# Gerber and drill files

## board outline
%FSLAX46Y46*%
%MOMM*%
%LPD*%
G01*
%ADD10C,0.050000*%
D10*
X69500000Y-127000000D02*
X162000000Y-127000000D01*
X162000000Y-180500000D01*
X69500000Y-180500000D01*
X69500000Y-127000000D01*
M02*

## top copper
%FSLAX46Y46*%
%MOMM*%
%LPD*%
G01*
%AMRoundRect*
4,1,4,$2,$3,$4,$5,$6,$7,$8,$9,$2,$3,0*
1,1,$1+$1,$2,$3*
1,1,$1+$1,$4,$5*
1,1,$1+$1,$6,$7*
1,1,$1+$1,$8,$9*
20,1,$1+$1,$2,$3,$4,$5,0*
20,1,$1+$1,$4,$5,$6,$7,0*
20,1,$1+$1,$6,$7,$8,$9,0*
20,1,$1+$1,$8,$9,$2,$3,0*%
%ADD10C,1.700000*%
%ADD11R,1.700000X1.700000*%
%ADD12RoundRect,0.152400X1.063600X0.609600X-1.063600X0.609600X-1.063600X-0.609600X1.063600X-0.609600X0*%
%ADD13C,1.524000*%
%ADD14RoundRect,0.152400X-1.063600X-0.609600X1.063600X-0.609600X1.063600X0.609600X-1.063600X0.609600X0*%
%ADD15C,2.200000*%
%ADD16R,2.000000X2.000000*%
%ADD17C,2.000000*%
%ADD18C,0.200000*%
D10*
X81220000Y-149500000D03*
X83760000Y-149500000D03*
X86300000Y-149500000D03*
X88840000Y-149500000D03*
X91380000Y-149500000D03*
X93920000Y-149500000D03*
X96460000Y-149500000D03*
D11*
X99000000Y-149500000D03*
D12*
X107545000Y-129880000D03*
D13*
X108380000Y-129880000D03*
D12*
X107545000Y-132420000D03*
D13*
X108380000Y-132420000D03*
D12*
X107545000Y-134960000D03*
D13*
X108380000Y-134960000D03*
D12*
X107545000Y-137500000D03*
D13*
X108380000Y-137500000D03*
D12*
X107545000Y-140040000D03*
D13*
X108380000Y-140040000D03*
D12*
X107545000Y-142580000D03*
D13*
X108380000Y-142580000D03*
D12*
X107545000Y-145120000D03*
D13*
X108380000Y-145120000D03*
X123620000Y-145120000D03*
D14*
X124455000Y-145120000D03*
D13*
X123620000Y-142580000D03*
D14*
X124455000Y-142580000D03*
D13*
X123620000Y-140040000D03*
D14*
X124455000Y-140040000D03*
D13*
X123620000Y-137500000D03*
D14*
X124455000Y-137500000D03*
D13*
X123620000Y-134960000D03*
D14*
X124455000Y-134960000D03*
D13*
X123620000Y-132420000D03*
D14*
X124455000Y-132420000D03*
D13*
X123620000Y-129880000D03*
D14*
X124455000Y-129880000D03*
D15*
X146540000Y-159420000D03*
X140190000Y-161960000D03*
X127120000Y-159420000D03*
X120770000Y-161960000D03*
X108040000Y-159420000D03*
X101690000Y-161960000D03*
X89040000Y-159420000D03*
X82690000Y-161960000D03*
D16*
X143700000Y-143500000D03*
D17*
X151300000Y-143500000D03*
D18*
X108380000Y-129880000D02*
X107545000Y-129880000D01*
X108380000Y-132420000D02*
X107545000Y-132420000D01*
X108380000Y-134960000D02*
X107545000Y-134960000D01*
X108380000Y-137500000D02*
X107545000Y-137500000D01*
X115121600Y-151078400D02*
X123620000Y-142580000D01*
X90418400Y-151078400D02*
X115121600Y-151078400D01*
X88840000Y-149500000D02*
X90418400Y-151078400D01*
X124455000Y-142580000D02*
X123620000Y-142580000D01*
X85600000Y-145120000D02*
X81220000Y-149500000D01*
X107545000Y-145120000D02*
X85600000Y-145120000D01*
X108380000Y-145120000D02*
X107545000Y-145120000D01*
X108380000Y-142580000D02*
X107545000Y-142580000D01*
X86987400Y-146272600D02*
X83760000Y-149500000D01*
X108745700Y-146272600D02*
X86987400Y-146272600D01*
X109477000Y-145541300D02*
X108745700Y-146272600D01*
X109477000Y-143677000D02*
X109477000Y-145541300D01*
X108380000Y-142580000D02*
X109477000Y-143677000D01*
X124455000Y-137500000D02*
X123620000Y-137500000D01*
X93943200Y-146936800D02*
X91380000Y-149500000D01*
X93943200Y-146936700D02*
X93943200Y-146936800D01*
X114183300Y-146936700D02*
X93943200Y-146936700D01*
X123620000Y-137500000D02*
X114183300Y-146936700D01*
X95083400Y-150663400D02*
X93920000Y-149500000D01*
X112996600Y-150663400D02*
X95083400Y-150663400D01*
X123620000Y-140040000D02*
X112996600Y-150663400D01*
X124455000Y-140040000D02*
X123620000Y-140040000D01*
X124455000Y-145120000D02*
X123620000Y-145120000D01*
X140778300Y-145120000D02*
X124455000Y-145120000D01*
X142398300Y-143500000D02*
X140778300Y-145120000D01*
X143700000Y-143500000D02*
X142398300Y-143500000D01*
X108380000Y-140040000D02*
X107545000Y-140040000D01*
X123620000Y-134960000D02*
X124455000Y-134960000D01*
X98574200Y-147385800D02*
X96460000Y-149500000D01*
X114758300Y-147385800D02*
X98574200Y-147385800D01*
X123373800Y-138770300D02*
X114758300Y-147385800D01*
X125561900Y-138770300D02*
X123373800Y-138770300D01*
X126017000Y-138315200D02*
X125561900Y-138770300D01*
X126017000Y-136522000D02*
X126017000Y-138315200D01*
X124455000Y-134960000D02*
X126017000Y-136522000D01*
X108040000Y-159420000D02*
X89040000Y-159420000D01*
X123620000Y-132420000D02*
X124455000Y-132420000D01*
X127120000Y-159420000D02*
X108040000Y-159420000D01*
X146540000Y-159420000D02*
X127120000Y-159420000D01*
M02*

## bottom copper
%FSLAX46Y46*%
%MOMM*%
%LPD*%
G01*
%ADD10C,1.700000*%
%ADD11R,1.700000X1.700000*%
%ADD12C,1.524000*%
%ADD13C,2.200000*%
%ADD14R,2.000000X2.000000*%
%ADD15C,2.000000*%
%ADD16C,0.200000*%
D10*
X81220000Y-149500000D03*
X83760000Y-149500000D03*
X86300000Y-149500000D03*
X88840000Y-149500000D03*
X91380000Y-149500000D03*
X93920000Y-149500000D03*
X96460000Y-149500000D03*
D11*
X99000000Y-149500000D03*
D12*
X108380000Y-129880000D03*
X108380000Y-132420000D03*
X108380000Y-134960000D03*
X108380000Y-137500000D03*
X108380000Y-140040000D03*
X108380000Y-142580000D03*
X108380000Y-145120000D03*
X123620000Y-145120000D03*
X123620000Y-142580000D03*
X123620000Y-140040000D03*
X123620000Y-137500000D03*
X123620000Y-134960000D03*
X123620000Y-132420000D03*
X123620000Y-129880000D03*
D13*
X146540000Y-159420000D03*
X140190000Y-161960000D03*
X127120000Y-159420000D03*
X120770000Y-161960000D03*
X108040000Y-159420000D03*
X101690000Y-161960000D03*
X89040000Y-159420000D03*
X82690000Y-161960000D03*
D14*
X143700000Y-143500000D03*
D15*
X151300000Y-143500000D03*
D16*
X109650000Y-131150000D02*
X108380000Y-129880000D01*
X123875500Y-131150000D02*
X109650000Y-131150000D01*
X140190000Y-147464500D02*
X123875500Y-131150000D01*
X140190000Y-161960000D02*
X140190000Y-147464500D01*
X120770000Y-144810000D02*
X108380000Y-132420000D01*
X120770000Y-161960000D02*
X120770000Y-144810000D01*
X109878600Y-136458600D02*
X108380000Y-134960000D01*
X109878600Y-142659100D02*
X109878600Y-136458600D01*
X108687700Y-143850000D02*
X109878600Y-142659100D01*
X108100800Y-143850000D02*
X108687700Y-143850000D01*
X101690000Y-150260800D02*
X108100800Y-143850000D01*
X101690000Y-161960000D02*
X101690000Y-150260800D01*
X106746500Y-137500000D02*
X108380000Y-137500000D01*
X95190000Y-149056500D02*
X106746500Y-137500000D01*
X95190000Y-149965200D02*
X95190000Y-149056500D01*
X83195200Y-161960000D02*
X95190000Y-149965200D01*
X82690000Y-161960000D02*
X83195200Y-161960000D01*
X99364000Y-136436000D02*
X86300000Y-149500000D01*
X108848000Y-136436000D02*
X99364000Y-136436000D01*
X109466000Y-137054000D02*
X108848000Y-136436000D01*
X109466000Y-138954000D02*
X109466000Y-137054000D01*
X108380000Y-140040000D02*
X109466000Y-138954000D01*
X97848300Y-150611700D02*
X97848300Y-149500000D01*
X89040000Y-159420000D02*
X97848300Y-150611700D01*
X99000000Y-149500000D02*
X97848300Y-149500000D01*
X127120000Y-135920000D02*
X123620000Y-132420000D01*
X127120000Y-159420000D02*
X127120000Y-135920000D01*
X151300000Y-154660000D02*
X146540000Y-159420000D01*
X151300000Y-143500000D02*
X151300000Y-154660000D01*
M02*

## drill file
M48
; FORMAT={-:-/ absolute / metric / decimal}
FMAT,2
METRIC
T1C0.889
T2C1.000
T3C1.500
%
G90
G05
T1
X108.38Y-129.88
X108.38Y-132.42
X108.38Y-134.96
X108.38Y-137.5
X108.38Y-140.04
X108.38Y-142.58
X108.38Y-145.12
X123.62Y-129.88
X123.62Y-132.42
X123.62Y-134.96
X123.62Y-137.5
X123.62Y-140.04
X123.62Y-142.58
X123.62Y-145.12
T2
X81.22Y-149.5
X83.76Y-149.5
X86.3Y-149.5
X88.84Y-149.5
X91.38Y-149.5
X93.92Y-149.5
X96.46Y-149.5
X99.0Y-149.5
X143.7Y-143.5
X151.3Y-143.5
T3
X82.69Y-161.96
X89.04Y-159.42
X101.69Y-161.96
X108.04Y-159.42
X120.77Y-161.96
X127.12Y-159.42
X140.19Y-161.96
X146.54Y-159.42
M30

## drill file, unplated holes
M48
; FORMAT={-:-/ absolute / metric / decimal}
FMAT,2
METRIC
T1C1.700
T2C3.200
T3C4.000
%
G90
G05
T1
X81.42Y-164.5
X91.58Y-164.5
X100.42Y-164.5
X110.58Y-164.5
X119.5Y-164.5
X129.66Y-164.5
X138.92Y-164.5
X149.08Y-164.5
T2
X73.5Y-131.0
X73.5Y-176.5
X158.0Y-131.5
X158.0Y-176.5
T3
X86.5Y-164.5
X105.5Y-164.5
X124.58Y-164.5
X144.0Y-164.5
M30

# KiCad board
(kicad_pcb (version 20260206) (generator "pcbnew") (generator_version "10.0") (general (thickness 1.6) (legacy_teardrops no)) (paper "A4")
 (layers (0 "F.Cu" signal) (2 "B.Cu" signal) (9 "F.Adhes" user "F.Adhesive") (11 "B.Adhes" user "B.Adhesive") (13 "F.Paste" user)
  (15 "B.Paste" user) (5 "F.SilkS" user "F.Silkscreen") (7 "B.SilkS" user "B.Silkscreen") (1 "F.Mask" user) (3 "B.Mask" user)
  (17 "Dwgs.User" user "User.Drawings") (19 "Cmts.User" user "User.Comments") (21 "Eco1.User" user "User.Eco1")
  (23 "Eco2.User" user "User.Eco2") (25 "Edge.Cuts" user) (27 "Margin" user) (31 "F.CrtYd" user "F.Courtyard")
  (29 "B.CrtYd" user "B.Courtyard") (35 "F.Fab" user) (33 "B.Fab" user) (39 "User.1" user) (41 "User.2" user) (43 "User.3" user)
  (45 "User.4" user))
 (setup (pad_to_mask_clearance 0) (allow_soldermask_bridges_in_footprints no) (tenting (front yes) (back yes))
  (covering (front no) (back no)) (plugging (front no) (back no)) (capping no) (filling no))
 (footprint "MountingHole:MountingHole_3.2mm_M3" (layer "F.Cu") (at 158 176.5)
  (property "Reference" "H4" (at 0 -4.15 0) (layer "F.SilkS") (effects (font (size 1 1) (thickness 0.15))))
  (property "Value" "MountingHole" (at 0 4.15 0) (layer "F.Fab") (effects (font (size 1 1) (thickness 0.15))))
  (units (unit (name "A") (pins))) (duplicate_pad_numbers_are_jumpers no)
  (pad "" np_thru_hole circle (at 0 0) (size 3.2 3.2) (drill 3.2) (layers "*.Cu" "*.Mask")))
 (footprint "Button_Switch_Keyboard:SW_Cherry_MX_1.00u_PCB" (layer "F.Cu") (at 127.12 159.42)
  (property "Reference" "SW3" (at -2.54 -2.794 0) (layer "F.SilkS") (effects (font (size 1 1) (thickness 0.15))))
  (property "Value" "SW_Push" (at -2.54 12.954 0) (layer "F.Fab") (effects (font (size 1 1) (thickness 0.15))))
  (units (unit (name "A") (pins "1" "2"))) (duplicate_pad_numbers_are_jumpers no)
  (pad "" np_thru_hole circle (at -7.62 5.08) (size 1.7 1.7) (drill 1.7) (layers "*.Cu" "*.Mask"))
  (pad "" np_thru_hole circle (at -2.54 5.08) (size 4 4) (drill 4) (layers "*.Cu" "*.Mask"))
  (pad "" np_thru_hole circle (at 2.54 5.08) (size 1.7 1.7) (drill 1.7) (layers "*.Cu" "*.Mask"))
  (pad "1" thru_hole circle (at 0 0) (size 2.2 2.2) (drill 1.5) (layers "*.Cu" "*.Mask") (remove_unused_layers no) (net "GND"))
  (pad "2" thru_hole circle (at -6.35 2.54) (size 2.2 2.2) (drill 1.5) (layers "*.Cu" "*.Mask") (remove_unused_layers no) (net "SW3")))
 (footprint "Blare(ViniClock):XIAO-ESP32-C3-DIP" (layer "F.Cu") (at 116 137.5 90)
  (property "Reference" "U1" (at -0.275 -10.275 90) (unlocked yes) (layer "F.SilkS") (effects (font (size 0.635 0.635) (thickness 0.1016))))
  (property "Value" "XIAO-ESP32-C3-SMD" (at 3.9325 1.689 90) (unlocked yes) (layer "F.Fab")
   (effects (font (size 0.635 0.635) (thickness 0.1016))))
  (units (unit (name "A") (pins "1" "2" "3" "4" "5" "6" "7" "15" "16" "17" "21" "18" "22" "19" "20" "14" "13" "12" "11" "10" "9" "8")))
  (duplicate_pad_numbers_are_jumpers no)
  (pad "1" smd roundrect (at 7.62 -8.455 180) (size 2.432 1.524) (layers "F.Cu" "F.Mask") (roundrect_rratio 0.1) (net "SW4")
   (thermal_bridge_angle 45))
  (pad "1" thru_hole circle (at 7.62 -7.62 180) (size 1.524 1.524) (drill 0.889) (layers "*.Cu" "*.Mask") (remove_unused_layers no)
   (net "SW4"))
  (pad "2" smd roundrect (at 5.08 -8.455 180) (size 2.432 1.524) (layers "F.Cu" "F.Mask") (roundrect_rratio 0.1) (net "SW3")
   (thermal_bridge_angle 45))
  (pad "2" thru_hole circle (at 5.08 -7.62 180) (size 1.524 1.524) (drill 0.889) (layers "*.Cu" "*.Mask") (remove_unused_layers no)
   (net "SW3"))
  (pad "3" smd roundrect (at 2.54 -8.455 180) (size 2.432 1.524) (layers "F.Cu" "F.Mask") (roundrect_rratio 0.1) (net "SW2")
   (thermal_bridge_angle 45))
  (pad "3" thru_hole circle (at 2.54 -7.62 180) (size 1.524 1.524) (drill 0.889) (layers "*.Cu" "*.Mask") (remove_unused_layers no)
   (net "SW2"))
  (pad "4" smd roundrect (at 0 -8.455 180) (size 2.432 1.524) (layers "F.Cu" "F.Mask") (roundrect_rratio 0.1) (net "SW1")
   (thermal_bridge_angle 45))
  (pad "4" thru_hole circle (at 0 -7.62 180) (size 1.524 1.524) (drill 0.889) (layers "*.Cu" "*.Mask") (remove_unused_layers no) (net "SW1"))
  (pad "5" smd roundrect (at -2.54 -8.455 180) (size 2.432 1.524) (layers "F.Cu" "F.Mask") (roundrect_rratio 0.1) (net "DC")
   (thermal_bridge_angle 45))
  (pad "5" thru_hole circle (at -2.54 -7.62 180) (size 1.524 1.524) (drill 0.889) (layers "*.Cu" "*.Mask") (remove_unused_layers no)
   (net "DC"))
  (pad "6" smd roundrect (at -5.08 -8.455 180) (size 2.432 1.524) (layers "F.Cu" "F.Mask") (roundrect_rratio 0.1) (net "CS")
   (thermal_bridge_angle 45))
  (pad "6" thru_hole circle (at -5.08 -7.62 180) (size 1.524 1.524) (drill 0.889) (layers "*.Cu" "*.Mask") (remove_unused_layers no)
   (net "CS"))
  (pad "7" smd roundrect (at -7.62 -8.455 180) (size 2.432 1.524) (layers "F.Cu" "F.Mask") (roundrect_rratio 0.1) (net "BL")
   (thermal_bridge_angle 45))
  (pad "7" thru_hole circle (at -7.62 -7.62 180) (size 1.524 1.524) (drill 0.889) (layers "*.Cu" "*.Mask") (remove_unused_layers no)
   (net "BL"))
  (pad "8" thru_hole circle (at -7.62 7.62) (size 1.524 1.524) (drill 0.889) (layers "*.Cu" "*.Mask") (remove_unused_layers no)
   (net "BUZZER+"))
  (pad "8" smd roundrect (at -7.62 8.455) (size 2.432 1.524) (layers "F.Cu" "F.Mask") (roundrect_rratio 0.1) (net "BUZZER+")
   (thermal_bridge_angle 45))
  (pad "9" thru_hole circle (at -5.08 7.62) (size 1.524 1.524) (drill 0.889) (layers "*.Cu" "*.Mask") (remove_unused_layers no) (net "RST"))
  (pad "9" smd roundrect (at -5.08 8.455) (size 2.432 1.524) (layers "F.Cu" "F.Mask") (roundrect_rratio 0.1) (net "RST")
   (thermal_bridge_angle 45))
  (pad "10" thru_hole circle (at -2.54 7.62) (size 1.524 1.524) (drill 0.889) (layers "*.Cu" "*.Mask") (remove_unused_layers no) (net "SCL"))
  (pad "10" smd roundrect (at -2.54 8.455) (size 2.432 1.524) (layers "F.Cu" "F.Mask") (roundrect_rratio 0.1) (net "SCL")
   (thermal_bridge_angle 45))
  (pad "11" thru_hole circle (at 0 7.62) (size 1.524 1.524) (drill 0.889) (layers "*.Cu" "*.Mask") (remove_unused_layers no) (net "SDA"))
  (pad "11" smd roundrect (at 0 8.455) (size 2.432 1.524) (layers "F.Cu" "F.Mask") (roundrect_rratio 0.1) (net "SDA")
   (thermal_bridge_angle 45))
  (pad "12" thru_hole circle (at 2.54 7.62) (size 1.524 1.524) (drill 0.889) (layers "*.Cu" "*.Mask") (remove_unused_layers no) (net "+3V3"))
  (pad "12" smd roundrect (at 2.54 8.455) (size 2.432 1.524) (layers "F.Cu" "F.Mask") (roundrect_rratio 0.1) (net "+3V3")
   (thermal_bridge_angle 45))
  (pad "13" thru_hole circle (at 5.08 7.62) (size 1.524 1.524) (drill 0.889) (layers "*.Cu" "*.Mask") (remove_unused_layers no) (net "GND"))
  (pad "13" smd roundrect (at 5.08 8.455) (size 2.432 1.524) (layers "F.Cu" "F.Mask") (roundrect_rratio 0.1) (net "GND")
   (thermal_bridge_angle 45))
  (pad "14" thru_hole circle (at 7.62 7.62) (size 1.524 1.524) (drill 0.889) (layers "*.Cu" "*.Mask") (remove_unused_layers no)
   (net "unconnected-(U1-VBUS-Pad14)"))
  (pad "14" smd roundrect (at 7.62 8.455) (size 2.432 1.524) (layers "F.Cu" "F.Mask") (roundrect_rratio 0.1)
   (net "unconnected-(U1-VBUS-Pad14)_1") (thermal_bridge_angle 45)))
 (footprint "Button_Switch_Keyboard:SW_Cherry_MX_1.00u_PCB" (layer "F.Cu") (at 89.04 159.42)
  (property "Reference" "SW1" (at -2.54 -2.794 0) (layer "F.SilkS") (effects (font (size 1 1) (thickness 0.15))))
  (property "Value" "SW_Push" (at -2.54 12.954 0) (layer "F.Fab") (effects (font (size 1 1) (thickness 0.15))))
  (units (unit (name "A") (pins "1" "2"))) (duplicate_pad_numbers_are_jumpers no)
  (pad "" np_thru_hole circle (at -7.62 5.08) (size 1.7 1.7) (drill 1.7) (layers "*.Cu" "*.Mask"))
  (pad "" np_thru_hole circle (at -2.54 5.08) (size 4 4) (drill 4) (layers "*.Cu" "*.Mask"))
  (pad "" np_thru_hole circle (at 2.54 5.08) (size 1.7 1.7) (drill 1.7) (layers "*.Cu" "*.Mask"))
  (pad "1" thru_hole circle (at 0 0) (size 2.2 2.2) (drill 1.5) (layers "*.Cu" "*.Mask") (remove_unused_layers no) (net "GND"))
  (pad "2" thru_hole circle (at -6.35 2.54) (size 2.2 2.2) (drill 1.5) (layers "*.Cu" "*.Mask") (remove_unused_layers no) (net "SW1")))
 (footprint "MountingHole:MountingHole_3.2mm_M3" (layer "F.Cu") (at 158 131.5)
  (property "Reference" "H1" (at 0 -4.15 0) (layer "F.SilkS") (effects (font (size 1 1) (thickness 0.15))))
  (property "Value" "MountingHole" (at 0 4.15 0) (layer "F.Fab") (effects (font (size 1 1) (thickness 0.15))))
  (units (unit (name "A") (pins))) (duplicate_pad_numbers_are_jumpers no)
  (pad "" np_thru_hole circle (at 0 0) (size 3.2 3.2) (drill 3.2) (layers "*.Cu" "*.Mask")))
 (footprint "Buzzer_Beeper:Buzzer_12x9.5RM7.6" (layer "F.Cu") (at 143.7 143.5)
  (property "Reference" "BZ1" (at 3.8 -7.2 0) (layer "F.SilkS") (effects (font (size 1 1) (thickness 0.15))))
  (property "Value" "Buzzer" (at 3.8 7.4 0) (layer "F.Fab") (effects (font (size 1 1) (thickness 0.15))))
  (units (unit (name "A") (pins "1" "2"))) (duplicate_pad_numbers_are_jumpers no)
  (pad "1" thru_hole rect (at 0 0) (size 2 2) (drill 1) (layers "*.Cu" "*.Mask") (remove_unused_layers no) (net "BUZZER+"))
  (pad "2" thru_hole circle (at 7.6 0) (size 2 2) (drill 1) (layers "*.Cu" "*.Mask") (remove_unused_layers no) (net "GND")))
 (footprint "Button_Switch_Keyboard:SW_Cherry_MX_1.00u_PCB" (layer "F.Cu") (at 108.04 159.42)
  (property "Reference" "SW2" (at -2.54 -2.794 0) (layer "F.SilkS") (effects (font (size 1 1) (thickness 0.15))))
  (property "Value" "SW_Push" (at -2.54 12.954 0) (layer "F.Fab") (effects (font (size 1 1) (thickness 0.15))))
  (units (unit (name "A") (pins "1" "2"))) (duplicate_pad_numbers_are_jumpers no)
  (pad "" np_thru_hole circle (at -7.62 5.08) (size 1.7 1.7) (drill 1.7) (layers "*.Cu" "*.Mask"))
  (pad "" np_thru_hole circle (at -2.54 5.08) (size 4 4) (drill 4) (layers "*.Cu" "*.Mask"))
  (pad "" np_thru_hole circle (at 2.54 5.08) (size 1.7 1.7) (drill 1.7) (layers "*.Cu" "*.Mask"))
  (pad "1" thru_hole circle (at 0 0) (size 2.2 2.2) (drill 1.5) (layers "*.Cu" "*.Mask") (remove_unused_layers no) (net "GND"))
  (pad "2" thru_hole circle (at -6.35 2.54) (size 2.2 2.2) (drill 1.5) (layers "*.Cu" "*.Mask") (remove_unused_layers no) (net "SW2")))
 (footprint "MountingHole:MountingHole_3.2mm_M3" (layer "F.Cu") (at 73.5 176.5)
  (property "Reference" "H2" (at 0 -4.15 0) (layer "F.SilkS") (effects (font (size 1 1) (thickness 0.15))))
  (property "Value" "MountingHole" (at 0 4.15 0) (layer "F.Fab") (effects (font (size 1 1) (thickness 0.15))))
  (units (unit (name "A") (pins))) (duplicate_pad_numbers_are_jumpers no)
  (pad "" np_thru_hole circle (at 0 0) (size 3.2 3.2) (drill 3.2) (layers "*.Cu" "*.Mask")))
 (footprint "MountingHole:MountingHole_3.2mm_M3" (layer "F.Cu") (at 73.5 131)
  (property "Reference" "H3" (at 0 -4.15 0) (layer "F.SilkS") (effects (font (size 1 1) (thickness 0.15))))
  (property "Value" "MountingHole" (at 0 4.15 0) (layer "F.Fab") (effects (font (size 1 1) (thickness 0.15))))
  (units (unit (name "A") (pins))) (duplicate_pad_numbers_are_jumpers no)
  (pad "" np_thru_hole circle (at 0 0) (size 3.2 3.2) (drill 3.2) (layers "*.Cu" "*.Mask")))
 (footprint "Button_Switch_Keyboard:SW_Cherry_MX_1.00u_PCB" (layer "F.Cu") (at 146.54 159.42)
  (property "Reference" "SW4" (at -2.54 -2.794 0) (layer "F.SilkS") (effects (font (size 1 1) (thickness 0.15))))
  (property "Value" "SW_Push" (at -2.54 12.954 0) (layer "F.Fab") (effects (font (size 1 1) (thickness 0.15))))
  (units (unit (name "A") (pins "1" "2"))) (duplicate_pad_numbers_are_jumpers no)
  (pad "" np_thru_hole circle (at -7.62 5.08) (size 1.7 1.7) (drill 1.7) (layers "*.Cu" "*.Mask"))
  (pad "" np_thru_hole circle (at -2.54 5.08) (size 4 4) (drill 4) (layers "*.Cu" "*.Mask"))
  (pad "" np_thru_hole circle (at 2.54 5.08) (size 1.7 1.7) (drill 1.7) (layers "*.Cu" "*.Mask"))
  (pad "1" thru_hole circle (at 0 0) (size 2.2 2.2) (drill 1.5) (layers "*.Cu" "*.Mask") (remove_unused_layers no) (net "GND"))
  (pad "2" thru_hole circle (at -6.35 2.54) (size 2.2 2.2) (drill 1.5) (layers "*.Cu" "*.Mask") (remove_unused_layers no) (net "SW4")))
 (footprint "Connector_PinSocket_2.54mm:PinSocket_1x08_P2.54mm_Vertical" (layer "B.Cu") (at 99 149.5 90)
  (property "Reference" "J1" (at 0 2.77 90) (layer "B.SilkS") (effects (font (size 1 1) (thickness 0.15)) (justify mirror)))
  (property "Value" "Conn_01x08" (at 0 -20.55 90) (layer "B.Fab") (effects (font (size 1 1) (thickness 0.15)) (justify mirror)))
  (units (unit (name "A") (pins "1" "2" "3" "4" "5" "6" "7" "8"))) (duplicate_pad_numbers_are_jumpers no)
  (pad "1" thru_hole rect (at 0 0 90) (size 1.7 1.7) (drill 1) (layers "*.Cu" "*.Mask") (remove_unused_layers no) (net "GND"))
  (pad "2" thru_hole circle (at 0 -2.54 90) (size 1.7 1.7) (drill 1) (layers "*.Cu" "*.Mask") (remove_unused_layers no) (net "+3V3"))
  (pad "3" thru_hole circle (at 0 -5.08 90) (size 1.7 1.7) (drill 1) (layers "*.Cu" "*.Mask") (remove_unused_layers no) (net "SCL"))
  (pad "4" thru_hole circle (at 0 -7.62 90) (size 1.7 1.7) (drill 1) (layers "*.Cu" "*.Mask") (remove_unused_layers no) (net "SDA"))
  (pad "5" thru_hole circle (at 0 -10.16 90) (size 1.7 1.7) (drill 1) (layers "*.Cu" "*.Mask") (remove_unused_layers no) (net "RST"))
  (pad "6" thru_hole circle (at 0 -12.7 90) (size 1.7 1.7) (drill 1) (layers "*.Cu" "*.Mask") (remove_unused_layers no) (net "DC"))
  (pad "7" thru_hole circle (at 0 -15.24 90) (size 1.7 1.7) (drill 1) (layers "*.Cu" "*.Mask") (remove_unused_layers no) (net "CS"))
  (pad "8" thru_hole circle (at 0 -17.78 90) (size 1.7 1.7) (drill 1) (layers "*.Cu" "*.Mask") (remove_unused_layers no) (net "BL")))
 (gr_rect (start 69.5 127) (end 162 180.5) (stroke (width 0.05) (type default)) (fill no) (layer "Edge.Cuts"))
 (segment (start 127.12 159.42) (end 108.04 159.42) (width 0.2) (layer "F.Cu") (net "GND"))
 (segment (start 146.54 159.42) (end 127.12 159.42) (width 0.2) (layer "F.Cu") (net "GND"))
 (segment (start 108.04 159.42) (end 89.04 159.42) (width 0.2) (layer "F.Cu") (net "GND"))
 (segment (start 123.62 132.42) (end 124.455 132.42) (width 0.2) (layer "F.Cu") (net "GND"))
 (segment (start 151.3 154.66) (end 146.54 159.42) (width 0.2) (layer "B.Cu") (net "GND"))
 (segment (start 127.12 135.92) (end 123.62 132.42) (width 0.2) (layer "B.Cu") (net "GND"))
 (segment (start 127.12 159.42) (end 127.12 135.92) (width 0.2) (layer "B.Cu") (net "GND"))
 (segment (start 89.04 159.42) (end 97.8483 150.6117) (width 0.2) (layer "B.Cu") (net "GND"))
 (segment (start 99 149.5) (end 97.8483 149.5) (width 0.2) (layer "B.Cu") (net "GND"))
 (segment (start 151.3 143.5) (end 151.3 154.66) (width 0.2) (layer "B.Cu") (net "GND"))
 (segment (start 97.8483 150.6117) (end 97.8483 149.5) (width 0.2) (layer "B.Cu") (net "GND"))
 (segment (start 108.38 132.42) (end 107.545 132.42) (width 0.2) (layer "F.Cu") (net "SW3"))
 (segment (start 120.77 144.81) (end 108.38 132.42) (width 0.2) (layer "B.Cu") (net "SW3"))
 (segment (start 120.77 161.96) (end 120.77 144.81) (width 0.2) (layer "B.Cu") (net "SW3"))
 (segment (start 108.38 129.88) (end 107.545 129.88) (width 0.2) (layer "F.Cu") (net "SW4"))
 (segment (start 109.65 131.15) (end 108.38 129.88) (width 0.2) (layer "B.Cu") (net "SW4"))
 (segment (start 140.19 147.4645) (end 123.8755 131.15) (width 0.2) (layer "B.Cu") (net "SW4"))
 (segment (start 123.8755 131.15) (end 109.65 131.15) (width 0.2) (layer "B.Cu") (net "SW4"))
 (segment (start 140.19 161.96) (end 140.19 147.4645) (width 0.2) (layer "B.Cu") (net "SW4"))
 (segment (start 108.38 134.96) (end 107.545 134.96) (width 0.2) (layer "F.Cu") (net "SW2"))
 (segment (start 108.6877 143.85) (end 109.8786 142.6591) (width 0.2) (layer "B.Cu") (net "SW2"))
 (segment (start 101.69 161.96) (end 101.69 150.2608) (width 0.2) (layer "B.Cu") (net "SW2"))
 (segment (start 109.8786 136.4586) (end 108.38 134.96) (width 0.2) (layer "B.Cu") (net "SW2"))
 (segment (start 108.1008 143.85) (end 108.6877 143.85) (width 0.2) (layer "B.Cu") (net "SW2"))
 (segment (start 101.69 150.2608) (end 108.1008 143.85) (width 0.2) (layer "B.Cu") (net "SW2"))
 (segment (start 109.8786 142.6591) (end 109.8786 136.4586) (width 0.2) (layer "B.Cu") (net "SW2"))
 (segment (start 108.38 137.5) (end 107.545 137.5) (width 0.2) (layer "F.Cu") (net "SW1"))
 (segment (start 95.19 149.9652) (end 95.19 149.0565) (width 0.2) (layer "B.Cu") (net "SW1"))
 (segment (start 83.1952 161.96) (end 95.19 149.9652) (width 0.2) (layer "B.Cu") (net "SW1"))
 (segment (start 95.19 149.0565) (end 106.7465 137.5) (width 0.2) (layer "B.Cu") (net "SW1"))
 (segment (start 82.69 161.96) (end 83.1952 161.96) (width 0.2) (layer "B.Cu") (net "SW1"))
 (segment (start 106.7465 137.5) (end 108.38 137.5) (width 0.2) (layer "B.Cu") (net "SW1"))
 (segment (start 108.38 140.04) (end 107.545 140.04) (width 0.2) (layer "F.Cu") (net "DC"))
 (segment (start 109.466 137.054) (end 108.848 136.436) (width 0.2) (layer "B.Cu") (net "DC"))
 (segment (start 108.38 140.04) (end 109.466 138.954) (width 0.2) (layer "B.Cu") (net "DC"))
 (segment (start 108.848 136.436) (end 99.364 136.436) (width 0.2) (layer "B.Cu") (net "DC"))
 (segment (start 109.466 138.954) (end 109.466 137.054) (width 0.2) (layer "B.Cu") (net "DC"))
 (segment (start 99.364 136.436) (end 86.3 149.5) (width 0.2) (layer "B.Cu") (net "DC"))
 (segment (start 108.38 142.58) (end 107.545 142.58) (width 0.2) (layer "F.Cu") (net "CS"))
 (segment (start 109.477 145.5413) (end 108.7457 146.2726) (width 0.2) (layer "F.Cu") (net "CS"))
 (segment (start 86.9874 146.2726) (end 83.76 149.5) (width 0.2) (layer "F.Cu") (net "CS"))
 (segment (start 108.7457 146.2726) (end 86.9874 146.2726) (width 0.2) (layer "F.Cu") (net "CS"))
 (segment (start 109.477 143.677) (end 109.477 145.5413) (width 0.2) (layer "F.Cu") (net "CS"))
 (segment (start 108.38 142.58) (end 109.477 143.677) (width 0.2) (layer "F.Cu") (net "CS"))
 (segment (start 107.545 145.12) (end 85.6 145.12) (width 0.2) (layer "F.Cu") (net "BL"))
 (segment (start 85.6 145.12) (end 81.22 149.5) (width 0.2) (layer "F.Cu") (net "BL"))
 (segment (start 108.38 145.12) (end 107.545 145.12) (width 0.2) (layer "F.Cu") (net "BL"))
 (segment (start 124.455 145.12) (end 123.62 145.12) (width 0.2) (layer "F.Cu") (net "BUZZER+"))
 (segment (start 142.3983 143.5) (end 140.7783 145.12) (width 0.2) (layer "F.Cu") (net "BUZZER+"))
 (segment (start 140.7783 145.12) (end 124.455 145.12) (width 0.2) (layer "F.Cu") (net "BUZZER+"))
 (segment (start 143.7 143.5) (end 142.3983 143.5) (width 0.2) (layer "F.Cu") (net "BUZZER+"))
 (segment (start 88.84 149.5) (end 90.4184 151.0784) (width 0.2) (layer "F.Cu") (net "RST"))
 (segment (start 124.455 142.58) (end 123.62 142.58) (width 0.2) (layer "F.Cu") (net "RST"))
 (segment (start 115.1216 151.0784) (end 123.62 142.58) (width 0.2) (layer "F.Cu") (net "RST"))
 (segment (start 90.4184 151.0784) (end 115.1216 151.0784) (width 0.2) (layer "F.Cu") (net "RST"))
 (segment (start 124.455 140.04) (end 123.62 140.04) (width 0.2) (layer "F.Cu") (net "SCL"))
 (segment (start 123.62 140.04) (end 112.9966 150.6634) (width 0.2) (layer "F.Cu") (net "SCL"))
 (segment (start 112.9966 150.6634) (end 95.0834 150.6634) (width 0.2) (layer "F.Cu") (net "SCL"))
 (segment (start 95.0834 150.6634) (end 93.92 149.5) (width 0.2) (layer "F.Cu") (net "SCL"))
 (segment (start 123.62 137.5) (end 114.1833 146.9367) (width 0.2) (layer "F.Cu") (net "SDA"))
 (segment (start 124.455 137.5) (end 123.62 137.5) (width 0.2) (layer "F.Cu") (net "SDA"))
 (segment (start 93.9432 146.9367) (end 93.9432 146.9368) (width 0.2) (layer "F.Cu") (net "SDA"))
 (segment (start 114.1833 146.9367) (end 93.9432 146.9367) (width 0.2) (layer "F.Cu") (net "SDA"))
 (segment (start 93.9432 146.9368) (end 91.38 149.5) (width 0.2) (layer "F.Cu") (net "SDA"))
 (segment (start 98.5742 147.3858) (end 96.46 149.5) (width 0.2) (layer "F.Cu") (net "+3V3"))
 (segment (start 114.7583 147.3858) (end 98.5742 147.3858) (width 0.2) (layer "F.Cu") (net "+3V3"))
 (segment (start 123.3738 138.7703) (end 114.7583 147.3858) (width 0.2) (layer "F.Cu") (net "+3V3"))
 (segment (start 123.62 134.96) (end 124.455 134.96) (width 0.2) (layer "F.Cu") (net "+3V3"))
 (segment (start 125.5619 138.7703) (end 123.3738 138.7703) (width 0.2) (layer "F.Cu") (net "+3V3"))
 (segment (start 124.455 134.96) (end 126.017 136.522) (width 0.2) (layer "F.Cu") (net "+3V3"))
 (segment (start 126.017 138.3152) (end 125.5619 138.7703) (width 0.2) (layer "F.Cu") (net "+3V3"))
 (segment (start 126.017 136.522) (end 126.017 138.3152) (width 0.2) (layer "F.Cu") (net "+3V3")))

